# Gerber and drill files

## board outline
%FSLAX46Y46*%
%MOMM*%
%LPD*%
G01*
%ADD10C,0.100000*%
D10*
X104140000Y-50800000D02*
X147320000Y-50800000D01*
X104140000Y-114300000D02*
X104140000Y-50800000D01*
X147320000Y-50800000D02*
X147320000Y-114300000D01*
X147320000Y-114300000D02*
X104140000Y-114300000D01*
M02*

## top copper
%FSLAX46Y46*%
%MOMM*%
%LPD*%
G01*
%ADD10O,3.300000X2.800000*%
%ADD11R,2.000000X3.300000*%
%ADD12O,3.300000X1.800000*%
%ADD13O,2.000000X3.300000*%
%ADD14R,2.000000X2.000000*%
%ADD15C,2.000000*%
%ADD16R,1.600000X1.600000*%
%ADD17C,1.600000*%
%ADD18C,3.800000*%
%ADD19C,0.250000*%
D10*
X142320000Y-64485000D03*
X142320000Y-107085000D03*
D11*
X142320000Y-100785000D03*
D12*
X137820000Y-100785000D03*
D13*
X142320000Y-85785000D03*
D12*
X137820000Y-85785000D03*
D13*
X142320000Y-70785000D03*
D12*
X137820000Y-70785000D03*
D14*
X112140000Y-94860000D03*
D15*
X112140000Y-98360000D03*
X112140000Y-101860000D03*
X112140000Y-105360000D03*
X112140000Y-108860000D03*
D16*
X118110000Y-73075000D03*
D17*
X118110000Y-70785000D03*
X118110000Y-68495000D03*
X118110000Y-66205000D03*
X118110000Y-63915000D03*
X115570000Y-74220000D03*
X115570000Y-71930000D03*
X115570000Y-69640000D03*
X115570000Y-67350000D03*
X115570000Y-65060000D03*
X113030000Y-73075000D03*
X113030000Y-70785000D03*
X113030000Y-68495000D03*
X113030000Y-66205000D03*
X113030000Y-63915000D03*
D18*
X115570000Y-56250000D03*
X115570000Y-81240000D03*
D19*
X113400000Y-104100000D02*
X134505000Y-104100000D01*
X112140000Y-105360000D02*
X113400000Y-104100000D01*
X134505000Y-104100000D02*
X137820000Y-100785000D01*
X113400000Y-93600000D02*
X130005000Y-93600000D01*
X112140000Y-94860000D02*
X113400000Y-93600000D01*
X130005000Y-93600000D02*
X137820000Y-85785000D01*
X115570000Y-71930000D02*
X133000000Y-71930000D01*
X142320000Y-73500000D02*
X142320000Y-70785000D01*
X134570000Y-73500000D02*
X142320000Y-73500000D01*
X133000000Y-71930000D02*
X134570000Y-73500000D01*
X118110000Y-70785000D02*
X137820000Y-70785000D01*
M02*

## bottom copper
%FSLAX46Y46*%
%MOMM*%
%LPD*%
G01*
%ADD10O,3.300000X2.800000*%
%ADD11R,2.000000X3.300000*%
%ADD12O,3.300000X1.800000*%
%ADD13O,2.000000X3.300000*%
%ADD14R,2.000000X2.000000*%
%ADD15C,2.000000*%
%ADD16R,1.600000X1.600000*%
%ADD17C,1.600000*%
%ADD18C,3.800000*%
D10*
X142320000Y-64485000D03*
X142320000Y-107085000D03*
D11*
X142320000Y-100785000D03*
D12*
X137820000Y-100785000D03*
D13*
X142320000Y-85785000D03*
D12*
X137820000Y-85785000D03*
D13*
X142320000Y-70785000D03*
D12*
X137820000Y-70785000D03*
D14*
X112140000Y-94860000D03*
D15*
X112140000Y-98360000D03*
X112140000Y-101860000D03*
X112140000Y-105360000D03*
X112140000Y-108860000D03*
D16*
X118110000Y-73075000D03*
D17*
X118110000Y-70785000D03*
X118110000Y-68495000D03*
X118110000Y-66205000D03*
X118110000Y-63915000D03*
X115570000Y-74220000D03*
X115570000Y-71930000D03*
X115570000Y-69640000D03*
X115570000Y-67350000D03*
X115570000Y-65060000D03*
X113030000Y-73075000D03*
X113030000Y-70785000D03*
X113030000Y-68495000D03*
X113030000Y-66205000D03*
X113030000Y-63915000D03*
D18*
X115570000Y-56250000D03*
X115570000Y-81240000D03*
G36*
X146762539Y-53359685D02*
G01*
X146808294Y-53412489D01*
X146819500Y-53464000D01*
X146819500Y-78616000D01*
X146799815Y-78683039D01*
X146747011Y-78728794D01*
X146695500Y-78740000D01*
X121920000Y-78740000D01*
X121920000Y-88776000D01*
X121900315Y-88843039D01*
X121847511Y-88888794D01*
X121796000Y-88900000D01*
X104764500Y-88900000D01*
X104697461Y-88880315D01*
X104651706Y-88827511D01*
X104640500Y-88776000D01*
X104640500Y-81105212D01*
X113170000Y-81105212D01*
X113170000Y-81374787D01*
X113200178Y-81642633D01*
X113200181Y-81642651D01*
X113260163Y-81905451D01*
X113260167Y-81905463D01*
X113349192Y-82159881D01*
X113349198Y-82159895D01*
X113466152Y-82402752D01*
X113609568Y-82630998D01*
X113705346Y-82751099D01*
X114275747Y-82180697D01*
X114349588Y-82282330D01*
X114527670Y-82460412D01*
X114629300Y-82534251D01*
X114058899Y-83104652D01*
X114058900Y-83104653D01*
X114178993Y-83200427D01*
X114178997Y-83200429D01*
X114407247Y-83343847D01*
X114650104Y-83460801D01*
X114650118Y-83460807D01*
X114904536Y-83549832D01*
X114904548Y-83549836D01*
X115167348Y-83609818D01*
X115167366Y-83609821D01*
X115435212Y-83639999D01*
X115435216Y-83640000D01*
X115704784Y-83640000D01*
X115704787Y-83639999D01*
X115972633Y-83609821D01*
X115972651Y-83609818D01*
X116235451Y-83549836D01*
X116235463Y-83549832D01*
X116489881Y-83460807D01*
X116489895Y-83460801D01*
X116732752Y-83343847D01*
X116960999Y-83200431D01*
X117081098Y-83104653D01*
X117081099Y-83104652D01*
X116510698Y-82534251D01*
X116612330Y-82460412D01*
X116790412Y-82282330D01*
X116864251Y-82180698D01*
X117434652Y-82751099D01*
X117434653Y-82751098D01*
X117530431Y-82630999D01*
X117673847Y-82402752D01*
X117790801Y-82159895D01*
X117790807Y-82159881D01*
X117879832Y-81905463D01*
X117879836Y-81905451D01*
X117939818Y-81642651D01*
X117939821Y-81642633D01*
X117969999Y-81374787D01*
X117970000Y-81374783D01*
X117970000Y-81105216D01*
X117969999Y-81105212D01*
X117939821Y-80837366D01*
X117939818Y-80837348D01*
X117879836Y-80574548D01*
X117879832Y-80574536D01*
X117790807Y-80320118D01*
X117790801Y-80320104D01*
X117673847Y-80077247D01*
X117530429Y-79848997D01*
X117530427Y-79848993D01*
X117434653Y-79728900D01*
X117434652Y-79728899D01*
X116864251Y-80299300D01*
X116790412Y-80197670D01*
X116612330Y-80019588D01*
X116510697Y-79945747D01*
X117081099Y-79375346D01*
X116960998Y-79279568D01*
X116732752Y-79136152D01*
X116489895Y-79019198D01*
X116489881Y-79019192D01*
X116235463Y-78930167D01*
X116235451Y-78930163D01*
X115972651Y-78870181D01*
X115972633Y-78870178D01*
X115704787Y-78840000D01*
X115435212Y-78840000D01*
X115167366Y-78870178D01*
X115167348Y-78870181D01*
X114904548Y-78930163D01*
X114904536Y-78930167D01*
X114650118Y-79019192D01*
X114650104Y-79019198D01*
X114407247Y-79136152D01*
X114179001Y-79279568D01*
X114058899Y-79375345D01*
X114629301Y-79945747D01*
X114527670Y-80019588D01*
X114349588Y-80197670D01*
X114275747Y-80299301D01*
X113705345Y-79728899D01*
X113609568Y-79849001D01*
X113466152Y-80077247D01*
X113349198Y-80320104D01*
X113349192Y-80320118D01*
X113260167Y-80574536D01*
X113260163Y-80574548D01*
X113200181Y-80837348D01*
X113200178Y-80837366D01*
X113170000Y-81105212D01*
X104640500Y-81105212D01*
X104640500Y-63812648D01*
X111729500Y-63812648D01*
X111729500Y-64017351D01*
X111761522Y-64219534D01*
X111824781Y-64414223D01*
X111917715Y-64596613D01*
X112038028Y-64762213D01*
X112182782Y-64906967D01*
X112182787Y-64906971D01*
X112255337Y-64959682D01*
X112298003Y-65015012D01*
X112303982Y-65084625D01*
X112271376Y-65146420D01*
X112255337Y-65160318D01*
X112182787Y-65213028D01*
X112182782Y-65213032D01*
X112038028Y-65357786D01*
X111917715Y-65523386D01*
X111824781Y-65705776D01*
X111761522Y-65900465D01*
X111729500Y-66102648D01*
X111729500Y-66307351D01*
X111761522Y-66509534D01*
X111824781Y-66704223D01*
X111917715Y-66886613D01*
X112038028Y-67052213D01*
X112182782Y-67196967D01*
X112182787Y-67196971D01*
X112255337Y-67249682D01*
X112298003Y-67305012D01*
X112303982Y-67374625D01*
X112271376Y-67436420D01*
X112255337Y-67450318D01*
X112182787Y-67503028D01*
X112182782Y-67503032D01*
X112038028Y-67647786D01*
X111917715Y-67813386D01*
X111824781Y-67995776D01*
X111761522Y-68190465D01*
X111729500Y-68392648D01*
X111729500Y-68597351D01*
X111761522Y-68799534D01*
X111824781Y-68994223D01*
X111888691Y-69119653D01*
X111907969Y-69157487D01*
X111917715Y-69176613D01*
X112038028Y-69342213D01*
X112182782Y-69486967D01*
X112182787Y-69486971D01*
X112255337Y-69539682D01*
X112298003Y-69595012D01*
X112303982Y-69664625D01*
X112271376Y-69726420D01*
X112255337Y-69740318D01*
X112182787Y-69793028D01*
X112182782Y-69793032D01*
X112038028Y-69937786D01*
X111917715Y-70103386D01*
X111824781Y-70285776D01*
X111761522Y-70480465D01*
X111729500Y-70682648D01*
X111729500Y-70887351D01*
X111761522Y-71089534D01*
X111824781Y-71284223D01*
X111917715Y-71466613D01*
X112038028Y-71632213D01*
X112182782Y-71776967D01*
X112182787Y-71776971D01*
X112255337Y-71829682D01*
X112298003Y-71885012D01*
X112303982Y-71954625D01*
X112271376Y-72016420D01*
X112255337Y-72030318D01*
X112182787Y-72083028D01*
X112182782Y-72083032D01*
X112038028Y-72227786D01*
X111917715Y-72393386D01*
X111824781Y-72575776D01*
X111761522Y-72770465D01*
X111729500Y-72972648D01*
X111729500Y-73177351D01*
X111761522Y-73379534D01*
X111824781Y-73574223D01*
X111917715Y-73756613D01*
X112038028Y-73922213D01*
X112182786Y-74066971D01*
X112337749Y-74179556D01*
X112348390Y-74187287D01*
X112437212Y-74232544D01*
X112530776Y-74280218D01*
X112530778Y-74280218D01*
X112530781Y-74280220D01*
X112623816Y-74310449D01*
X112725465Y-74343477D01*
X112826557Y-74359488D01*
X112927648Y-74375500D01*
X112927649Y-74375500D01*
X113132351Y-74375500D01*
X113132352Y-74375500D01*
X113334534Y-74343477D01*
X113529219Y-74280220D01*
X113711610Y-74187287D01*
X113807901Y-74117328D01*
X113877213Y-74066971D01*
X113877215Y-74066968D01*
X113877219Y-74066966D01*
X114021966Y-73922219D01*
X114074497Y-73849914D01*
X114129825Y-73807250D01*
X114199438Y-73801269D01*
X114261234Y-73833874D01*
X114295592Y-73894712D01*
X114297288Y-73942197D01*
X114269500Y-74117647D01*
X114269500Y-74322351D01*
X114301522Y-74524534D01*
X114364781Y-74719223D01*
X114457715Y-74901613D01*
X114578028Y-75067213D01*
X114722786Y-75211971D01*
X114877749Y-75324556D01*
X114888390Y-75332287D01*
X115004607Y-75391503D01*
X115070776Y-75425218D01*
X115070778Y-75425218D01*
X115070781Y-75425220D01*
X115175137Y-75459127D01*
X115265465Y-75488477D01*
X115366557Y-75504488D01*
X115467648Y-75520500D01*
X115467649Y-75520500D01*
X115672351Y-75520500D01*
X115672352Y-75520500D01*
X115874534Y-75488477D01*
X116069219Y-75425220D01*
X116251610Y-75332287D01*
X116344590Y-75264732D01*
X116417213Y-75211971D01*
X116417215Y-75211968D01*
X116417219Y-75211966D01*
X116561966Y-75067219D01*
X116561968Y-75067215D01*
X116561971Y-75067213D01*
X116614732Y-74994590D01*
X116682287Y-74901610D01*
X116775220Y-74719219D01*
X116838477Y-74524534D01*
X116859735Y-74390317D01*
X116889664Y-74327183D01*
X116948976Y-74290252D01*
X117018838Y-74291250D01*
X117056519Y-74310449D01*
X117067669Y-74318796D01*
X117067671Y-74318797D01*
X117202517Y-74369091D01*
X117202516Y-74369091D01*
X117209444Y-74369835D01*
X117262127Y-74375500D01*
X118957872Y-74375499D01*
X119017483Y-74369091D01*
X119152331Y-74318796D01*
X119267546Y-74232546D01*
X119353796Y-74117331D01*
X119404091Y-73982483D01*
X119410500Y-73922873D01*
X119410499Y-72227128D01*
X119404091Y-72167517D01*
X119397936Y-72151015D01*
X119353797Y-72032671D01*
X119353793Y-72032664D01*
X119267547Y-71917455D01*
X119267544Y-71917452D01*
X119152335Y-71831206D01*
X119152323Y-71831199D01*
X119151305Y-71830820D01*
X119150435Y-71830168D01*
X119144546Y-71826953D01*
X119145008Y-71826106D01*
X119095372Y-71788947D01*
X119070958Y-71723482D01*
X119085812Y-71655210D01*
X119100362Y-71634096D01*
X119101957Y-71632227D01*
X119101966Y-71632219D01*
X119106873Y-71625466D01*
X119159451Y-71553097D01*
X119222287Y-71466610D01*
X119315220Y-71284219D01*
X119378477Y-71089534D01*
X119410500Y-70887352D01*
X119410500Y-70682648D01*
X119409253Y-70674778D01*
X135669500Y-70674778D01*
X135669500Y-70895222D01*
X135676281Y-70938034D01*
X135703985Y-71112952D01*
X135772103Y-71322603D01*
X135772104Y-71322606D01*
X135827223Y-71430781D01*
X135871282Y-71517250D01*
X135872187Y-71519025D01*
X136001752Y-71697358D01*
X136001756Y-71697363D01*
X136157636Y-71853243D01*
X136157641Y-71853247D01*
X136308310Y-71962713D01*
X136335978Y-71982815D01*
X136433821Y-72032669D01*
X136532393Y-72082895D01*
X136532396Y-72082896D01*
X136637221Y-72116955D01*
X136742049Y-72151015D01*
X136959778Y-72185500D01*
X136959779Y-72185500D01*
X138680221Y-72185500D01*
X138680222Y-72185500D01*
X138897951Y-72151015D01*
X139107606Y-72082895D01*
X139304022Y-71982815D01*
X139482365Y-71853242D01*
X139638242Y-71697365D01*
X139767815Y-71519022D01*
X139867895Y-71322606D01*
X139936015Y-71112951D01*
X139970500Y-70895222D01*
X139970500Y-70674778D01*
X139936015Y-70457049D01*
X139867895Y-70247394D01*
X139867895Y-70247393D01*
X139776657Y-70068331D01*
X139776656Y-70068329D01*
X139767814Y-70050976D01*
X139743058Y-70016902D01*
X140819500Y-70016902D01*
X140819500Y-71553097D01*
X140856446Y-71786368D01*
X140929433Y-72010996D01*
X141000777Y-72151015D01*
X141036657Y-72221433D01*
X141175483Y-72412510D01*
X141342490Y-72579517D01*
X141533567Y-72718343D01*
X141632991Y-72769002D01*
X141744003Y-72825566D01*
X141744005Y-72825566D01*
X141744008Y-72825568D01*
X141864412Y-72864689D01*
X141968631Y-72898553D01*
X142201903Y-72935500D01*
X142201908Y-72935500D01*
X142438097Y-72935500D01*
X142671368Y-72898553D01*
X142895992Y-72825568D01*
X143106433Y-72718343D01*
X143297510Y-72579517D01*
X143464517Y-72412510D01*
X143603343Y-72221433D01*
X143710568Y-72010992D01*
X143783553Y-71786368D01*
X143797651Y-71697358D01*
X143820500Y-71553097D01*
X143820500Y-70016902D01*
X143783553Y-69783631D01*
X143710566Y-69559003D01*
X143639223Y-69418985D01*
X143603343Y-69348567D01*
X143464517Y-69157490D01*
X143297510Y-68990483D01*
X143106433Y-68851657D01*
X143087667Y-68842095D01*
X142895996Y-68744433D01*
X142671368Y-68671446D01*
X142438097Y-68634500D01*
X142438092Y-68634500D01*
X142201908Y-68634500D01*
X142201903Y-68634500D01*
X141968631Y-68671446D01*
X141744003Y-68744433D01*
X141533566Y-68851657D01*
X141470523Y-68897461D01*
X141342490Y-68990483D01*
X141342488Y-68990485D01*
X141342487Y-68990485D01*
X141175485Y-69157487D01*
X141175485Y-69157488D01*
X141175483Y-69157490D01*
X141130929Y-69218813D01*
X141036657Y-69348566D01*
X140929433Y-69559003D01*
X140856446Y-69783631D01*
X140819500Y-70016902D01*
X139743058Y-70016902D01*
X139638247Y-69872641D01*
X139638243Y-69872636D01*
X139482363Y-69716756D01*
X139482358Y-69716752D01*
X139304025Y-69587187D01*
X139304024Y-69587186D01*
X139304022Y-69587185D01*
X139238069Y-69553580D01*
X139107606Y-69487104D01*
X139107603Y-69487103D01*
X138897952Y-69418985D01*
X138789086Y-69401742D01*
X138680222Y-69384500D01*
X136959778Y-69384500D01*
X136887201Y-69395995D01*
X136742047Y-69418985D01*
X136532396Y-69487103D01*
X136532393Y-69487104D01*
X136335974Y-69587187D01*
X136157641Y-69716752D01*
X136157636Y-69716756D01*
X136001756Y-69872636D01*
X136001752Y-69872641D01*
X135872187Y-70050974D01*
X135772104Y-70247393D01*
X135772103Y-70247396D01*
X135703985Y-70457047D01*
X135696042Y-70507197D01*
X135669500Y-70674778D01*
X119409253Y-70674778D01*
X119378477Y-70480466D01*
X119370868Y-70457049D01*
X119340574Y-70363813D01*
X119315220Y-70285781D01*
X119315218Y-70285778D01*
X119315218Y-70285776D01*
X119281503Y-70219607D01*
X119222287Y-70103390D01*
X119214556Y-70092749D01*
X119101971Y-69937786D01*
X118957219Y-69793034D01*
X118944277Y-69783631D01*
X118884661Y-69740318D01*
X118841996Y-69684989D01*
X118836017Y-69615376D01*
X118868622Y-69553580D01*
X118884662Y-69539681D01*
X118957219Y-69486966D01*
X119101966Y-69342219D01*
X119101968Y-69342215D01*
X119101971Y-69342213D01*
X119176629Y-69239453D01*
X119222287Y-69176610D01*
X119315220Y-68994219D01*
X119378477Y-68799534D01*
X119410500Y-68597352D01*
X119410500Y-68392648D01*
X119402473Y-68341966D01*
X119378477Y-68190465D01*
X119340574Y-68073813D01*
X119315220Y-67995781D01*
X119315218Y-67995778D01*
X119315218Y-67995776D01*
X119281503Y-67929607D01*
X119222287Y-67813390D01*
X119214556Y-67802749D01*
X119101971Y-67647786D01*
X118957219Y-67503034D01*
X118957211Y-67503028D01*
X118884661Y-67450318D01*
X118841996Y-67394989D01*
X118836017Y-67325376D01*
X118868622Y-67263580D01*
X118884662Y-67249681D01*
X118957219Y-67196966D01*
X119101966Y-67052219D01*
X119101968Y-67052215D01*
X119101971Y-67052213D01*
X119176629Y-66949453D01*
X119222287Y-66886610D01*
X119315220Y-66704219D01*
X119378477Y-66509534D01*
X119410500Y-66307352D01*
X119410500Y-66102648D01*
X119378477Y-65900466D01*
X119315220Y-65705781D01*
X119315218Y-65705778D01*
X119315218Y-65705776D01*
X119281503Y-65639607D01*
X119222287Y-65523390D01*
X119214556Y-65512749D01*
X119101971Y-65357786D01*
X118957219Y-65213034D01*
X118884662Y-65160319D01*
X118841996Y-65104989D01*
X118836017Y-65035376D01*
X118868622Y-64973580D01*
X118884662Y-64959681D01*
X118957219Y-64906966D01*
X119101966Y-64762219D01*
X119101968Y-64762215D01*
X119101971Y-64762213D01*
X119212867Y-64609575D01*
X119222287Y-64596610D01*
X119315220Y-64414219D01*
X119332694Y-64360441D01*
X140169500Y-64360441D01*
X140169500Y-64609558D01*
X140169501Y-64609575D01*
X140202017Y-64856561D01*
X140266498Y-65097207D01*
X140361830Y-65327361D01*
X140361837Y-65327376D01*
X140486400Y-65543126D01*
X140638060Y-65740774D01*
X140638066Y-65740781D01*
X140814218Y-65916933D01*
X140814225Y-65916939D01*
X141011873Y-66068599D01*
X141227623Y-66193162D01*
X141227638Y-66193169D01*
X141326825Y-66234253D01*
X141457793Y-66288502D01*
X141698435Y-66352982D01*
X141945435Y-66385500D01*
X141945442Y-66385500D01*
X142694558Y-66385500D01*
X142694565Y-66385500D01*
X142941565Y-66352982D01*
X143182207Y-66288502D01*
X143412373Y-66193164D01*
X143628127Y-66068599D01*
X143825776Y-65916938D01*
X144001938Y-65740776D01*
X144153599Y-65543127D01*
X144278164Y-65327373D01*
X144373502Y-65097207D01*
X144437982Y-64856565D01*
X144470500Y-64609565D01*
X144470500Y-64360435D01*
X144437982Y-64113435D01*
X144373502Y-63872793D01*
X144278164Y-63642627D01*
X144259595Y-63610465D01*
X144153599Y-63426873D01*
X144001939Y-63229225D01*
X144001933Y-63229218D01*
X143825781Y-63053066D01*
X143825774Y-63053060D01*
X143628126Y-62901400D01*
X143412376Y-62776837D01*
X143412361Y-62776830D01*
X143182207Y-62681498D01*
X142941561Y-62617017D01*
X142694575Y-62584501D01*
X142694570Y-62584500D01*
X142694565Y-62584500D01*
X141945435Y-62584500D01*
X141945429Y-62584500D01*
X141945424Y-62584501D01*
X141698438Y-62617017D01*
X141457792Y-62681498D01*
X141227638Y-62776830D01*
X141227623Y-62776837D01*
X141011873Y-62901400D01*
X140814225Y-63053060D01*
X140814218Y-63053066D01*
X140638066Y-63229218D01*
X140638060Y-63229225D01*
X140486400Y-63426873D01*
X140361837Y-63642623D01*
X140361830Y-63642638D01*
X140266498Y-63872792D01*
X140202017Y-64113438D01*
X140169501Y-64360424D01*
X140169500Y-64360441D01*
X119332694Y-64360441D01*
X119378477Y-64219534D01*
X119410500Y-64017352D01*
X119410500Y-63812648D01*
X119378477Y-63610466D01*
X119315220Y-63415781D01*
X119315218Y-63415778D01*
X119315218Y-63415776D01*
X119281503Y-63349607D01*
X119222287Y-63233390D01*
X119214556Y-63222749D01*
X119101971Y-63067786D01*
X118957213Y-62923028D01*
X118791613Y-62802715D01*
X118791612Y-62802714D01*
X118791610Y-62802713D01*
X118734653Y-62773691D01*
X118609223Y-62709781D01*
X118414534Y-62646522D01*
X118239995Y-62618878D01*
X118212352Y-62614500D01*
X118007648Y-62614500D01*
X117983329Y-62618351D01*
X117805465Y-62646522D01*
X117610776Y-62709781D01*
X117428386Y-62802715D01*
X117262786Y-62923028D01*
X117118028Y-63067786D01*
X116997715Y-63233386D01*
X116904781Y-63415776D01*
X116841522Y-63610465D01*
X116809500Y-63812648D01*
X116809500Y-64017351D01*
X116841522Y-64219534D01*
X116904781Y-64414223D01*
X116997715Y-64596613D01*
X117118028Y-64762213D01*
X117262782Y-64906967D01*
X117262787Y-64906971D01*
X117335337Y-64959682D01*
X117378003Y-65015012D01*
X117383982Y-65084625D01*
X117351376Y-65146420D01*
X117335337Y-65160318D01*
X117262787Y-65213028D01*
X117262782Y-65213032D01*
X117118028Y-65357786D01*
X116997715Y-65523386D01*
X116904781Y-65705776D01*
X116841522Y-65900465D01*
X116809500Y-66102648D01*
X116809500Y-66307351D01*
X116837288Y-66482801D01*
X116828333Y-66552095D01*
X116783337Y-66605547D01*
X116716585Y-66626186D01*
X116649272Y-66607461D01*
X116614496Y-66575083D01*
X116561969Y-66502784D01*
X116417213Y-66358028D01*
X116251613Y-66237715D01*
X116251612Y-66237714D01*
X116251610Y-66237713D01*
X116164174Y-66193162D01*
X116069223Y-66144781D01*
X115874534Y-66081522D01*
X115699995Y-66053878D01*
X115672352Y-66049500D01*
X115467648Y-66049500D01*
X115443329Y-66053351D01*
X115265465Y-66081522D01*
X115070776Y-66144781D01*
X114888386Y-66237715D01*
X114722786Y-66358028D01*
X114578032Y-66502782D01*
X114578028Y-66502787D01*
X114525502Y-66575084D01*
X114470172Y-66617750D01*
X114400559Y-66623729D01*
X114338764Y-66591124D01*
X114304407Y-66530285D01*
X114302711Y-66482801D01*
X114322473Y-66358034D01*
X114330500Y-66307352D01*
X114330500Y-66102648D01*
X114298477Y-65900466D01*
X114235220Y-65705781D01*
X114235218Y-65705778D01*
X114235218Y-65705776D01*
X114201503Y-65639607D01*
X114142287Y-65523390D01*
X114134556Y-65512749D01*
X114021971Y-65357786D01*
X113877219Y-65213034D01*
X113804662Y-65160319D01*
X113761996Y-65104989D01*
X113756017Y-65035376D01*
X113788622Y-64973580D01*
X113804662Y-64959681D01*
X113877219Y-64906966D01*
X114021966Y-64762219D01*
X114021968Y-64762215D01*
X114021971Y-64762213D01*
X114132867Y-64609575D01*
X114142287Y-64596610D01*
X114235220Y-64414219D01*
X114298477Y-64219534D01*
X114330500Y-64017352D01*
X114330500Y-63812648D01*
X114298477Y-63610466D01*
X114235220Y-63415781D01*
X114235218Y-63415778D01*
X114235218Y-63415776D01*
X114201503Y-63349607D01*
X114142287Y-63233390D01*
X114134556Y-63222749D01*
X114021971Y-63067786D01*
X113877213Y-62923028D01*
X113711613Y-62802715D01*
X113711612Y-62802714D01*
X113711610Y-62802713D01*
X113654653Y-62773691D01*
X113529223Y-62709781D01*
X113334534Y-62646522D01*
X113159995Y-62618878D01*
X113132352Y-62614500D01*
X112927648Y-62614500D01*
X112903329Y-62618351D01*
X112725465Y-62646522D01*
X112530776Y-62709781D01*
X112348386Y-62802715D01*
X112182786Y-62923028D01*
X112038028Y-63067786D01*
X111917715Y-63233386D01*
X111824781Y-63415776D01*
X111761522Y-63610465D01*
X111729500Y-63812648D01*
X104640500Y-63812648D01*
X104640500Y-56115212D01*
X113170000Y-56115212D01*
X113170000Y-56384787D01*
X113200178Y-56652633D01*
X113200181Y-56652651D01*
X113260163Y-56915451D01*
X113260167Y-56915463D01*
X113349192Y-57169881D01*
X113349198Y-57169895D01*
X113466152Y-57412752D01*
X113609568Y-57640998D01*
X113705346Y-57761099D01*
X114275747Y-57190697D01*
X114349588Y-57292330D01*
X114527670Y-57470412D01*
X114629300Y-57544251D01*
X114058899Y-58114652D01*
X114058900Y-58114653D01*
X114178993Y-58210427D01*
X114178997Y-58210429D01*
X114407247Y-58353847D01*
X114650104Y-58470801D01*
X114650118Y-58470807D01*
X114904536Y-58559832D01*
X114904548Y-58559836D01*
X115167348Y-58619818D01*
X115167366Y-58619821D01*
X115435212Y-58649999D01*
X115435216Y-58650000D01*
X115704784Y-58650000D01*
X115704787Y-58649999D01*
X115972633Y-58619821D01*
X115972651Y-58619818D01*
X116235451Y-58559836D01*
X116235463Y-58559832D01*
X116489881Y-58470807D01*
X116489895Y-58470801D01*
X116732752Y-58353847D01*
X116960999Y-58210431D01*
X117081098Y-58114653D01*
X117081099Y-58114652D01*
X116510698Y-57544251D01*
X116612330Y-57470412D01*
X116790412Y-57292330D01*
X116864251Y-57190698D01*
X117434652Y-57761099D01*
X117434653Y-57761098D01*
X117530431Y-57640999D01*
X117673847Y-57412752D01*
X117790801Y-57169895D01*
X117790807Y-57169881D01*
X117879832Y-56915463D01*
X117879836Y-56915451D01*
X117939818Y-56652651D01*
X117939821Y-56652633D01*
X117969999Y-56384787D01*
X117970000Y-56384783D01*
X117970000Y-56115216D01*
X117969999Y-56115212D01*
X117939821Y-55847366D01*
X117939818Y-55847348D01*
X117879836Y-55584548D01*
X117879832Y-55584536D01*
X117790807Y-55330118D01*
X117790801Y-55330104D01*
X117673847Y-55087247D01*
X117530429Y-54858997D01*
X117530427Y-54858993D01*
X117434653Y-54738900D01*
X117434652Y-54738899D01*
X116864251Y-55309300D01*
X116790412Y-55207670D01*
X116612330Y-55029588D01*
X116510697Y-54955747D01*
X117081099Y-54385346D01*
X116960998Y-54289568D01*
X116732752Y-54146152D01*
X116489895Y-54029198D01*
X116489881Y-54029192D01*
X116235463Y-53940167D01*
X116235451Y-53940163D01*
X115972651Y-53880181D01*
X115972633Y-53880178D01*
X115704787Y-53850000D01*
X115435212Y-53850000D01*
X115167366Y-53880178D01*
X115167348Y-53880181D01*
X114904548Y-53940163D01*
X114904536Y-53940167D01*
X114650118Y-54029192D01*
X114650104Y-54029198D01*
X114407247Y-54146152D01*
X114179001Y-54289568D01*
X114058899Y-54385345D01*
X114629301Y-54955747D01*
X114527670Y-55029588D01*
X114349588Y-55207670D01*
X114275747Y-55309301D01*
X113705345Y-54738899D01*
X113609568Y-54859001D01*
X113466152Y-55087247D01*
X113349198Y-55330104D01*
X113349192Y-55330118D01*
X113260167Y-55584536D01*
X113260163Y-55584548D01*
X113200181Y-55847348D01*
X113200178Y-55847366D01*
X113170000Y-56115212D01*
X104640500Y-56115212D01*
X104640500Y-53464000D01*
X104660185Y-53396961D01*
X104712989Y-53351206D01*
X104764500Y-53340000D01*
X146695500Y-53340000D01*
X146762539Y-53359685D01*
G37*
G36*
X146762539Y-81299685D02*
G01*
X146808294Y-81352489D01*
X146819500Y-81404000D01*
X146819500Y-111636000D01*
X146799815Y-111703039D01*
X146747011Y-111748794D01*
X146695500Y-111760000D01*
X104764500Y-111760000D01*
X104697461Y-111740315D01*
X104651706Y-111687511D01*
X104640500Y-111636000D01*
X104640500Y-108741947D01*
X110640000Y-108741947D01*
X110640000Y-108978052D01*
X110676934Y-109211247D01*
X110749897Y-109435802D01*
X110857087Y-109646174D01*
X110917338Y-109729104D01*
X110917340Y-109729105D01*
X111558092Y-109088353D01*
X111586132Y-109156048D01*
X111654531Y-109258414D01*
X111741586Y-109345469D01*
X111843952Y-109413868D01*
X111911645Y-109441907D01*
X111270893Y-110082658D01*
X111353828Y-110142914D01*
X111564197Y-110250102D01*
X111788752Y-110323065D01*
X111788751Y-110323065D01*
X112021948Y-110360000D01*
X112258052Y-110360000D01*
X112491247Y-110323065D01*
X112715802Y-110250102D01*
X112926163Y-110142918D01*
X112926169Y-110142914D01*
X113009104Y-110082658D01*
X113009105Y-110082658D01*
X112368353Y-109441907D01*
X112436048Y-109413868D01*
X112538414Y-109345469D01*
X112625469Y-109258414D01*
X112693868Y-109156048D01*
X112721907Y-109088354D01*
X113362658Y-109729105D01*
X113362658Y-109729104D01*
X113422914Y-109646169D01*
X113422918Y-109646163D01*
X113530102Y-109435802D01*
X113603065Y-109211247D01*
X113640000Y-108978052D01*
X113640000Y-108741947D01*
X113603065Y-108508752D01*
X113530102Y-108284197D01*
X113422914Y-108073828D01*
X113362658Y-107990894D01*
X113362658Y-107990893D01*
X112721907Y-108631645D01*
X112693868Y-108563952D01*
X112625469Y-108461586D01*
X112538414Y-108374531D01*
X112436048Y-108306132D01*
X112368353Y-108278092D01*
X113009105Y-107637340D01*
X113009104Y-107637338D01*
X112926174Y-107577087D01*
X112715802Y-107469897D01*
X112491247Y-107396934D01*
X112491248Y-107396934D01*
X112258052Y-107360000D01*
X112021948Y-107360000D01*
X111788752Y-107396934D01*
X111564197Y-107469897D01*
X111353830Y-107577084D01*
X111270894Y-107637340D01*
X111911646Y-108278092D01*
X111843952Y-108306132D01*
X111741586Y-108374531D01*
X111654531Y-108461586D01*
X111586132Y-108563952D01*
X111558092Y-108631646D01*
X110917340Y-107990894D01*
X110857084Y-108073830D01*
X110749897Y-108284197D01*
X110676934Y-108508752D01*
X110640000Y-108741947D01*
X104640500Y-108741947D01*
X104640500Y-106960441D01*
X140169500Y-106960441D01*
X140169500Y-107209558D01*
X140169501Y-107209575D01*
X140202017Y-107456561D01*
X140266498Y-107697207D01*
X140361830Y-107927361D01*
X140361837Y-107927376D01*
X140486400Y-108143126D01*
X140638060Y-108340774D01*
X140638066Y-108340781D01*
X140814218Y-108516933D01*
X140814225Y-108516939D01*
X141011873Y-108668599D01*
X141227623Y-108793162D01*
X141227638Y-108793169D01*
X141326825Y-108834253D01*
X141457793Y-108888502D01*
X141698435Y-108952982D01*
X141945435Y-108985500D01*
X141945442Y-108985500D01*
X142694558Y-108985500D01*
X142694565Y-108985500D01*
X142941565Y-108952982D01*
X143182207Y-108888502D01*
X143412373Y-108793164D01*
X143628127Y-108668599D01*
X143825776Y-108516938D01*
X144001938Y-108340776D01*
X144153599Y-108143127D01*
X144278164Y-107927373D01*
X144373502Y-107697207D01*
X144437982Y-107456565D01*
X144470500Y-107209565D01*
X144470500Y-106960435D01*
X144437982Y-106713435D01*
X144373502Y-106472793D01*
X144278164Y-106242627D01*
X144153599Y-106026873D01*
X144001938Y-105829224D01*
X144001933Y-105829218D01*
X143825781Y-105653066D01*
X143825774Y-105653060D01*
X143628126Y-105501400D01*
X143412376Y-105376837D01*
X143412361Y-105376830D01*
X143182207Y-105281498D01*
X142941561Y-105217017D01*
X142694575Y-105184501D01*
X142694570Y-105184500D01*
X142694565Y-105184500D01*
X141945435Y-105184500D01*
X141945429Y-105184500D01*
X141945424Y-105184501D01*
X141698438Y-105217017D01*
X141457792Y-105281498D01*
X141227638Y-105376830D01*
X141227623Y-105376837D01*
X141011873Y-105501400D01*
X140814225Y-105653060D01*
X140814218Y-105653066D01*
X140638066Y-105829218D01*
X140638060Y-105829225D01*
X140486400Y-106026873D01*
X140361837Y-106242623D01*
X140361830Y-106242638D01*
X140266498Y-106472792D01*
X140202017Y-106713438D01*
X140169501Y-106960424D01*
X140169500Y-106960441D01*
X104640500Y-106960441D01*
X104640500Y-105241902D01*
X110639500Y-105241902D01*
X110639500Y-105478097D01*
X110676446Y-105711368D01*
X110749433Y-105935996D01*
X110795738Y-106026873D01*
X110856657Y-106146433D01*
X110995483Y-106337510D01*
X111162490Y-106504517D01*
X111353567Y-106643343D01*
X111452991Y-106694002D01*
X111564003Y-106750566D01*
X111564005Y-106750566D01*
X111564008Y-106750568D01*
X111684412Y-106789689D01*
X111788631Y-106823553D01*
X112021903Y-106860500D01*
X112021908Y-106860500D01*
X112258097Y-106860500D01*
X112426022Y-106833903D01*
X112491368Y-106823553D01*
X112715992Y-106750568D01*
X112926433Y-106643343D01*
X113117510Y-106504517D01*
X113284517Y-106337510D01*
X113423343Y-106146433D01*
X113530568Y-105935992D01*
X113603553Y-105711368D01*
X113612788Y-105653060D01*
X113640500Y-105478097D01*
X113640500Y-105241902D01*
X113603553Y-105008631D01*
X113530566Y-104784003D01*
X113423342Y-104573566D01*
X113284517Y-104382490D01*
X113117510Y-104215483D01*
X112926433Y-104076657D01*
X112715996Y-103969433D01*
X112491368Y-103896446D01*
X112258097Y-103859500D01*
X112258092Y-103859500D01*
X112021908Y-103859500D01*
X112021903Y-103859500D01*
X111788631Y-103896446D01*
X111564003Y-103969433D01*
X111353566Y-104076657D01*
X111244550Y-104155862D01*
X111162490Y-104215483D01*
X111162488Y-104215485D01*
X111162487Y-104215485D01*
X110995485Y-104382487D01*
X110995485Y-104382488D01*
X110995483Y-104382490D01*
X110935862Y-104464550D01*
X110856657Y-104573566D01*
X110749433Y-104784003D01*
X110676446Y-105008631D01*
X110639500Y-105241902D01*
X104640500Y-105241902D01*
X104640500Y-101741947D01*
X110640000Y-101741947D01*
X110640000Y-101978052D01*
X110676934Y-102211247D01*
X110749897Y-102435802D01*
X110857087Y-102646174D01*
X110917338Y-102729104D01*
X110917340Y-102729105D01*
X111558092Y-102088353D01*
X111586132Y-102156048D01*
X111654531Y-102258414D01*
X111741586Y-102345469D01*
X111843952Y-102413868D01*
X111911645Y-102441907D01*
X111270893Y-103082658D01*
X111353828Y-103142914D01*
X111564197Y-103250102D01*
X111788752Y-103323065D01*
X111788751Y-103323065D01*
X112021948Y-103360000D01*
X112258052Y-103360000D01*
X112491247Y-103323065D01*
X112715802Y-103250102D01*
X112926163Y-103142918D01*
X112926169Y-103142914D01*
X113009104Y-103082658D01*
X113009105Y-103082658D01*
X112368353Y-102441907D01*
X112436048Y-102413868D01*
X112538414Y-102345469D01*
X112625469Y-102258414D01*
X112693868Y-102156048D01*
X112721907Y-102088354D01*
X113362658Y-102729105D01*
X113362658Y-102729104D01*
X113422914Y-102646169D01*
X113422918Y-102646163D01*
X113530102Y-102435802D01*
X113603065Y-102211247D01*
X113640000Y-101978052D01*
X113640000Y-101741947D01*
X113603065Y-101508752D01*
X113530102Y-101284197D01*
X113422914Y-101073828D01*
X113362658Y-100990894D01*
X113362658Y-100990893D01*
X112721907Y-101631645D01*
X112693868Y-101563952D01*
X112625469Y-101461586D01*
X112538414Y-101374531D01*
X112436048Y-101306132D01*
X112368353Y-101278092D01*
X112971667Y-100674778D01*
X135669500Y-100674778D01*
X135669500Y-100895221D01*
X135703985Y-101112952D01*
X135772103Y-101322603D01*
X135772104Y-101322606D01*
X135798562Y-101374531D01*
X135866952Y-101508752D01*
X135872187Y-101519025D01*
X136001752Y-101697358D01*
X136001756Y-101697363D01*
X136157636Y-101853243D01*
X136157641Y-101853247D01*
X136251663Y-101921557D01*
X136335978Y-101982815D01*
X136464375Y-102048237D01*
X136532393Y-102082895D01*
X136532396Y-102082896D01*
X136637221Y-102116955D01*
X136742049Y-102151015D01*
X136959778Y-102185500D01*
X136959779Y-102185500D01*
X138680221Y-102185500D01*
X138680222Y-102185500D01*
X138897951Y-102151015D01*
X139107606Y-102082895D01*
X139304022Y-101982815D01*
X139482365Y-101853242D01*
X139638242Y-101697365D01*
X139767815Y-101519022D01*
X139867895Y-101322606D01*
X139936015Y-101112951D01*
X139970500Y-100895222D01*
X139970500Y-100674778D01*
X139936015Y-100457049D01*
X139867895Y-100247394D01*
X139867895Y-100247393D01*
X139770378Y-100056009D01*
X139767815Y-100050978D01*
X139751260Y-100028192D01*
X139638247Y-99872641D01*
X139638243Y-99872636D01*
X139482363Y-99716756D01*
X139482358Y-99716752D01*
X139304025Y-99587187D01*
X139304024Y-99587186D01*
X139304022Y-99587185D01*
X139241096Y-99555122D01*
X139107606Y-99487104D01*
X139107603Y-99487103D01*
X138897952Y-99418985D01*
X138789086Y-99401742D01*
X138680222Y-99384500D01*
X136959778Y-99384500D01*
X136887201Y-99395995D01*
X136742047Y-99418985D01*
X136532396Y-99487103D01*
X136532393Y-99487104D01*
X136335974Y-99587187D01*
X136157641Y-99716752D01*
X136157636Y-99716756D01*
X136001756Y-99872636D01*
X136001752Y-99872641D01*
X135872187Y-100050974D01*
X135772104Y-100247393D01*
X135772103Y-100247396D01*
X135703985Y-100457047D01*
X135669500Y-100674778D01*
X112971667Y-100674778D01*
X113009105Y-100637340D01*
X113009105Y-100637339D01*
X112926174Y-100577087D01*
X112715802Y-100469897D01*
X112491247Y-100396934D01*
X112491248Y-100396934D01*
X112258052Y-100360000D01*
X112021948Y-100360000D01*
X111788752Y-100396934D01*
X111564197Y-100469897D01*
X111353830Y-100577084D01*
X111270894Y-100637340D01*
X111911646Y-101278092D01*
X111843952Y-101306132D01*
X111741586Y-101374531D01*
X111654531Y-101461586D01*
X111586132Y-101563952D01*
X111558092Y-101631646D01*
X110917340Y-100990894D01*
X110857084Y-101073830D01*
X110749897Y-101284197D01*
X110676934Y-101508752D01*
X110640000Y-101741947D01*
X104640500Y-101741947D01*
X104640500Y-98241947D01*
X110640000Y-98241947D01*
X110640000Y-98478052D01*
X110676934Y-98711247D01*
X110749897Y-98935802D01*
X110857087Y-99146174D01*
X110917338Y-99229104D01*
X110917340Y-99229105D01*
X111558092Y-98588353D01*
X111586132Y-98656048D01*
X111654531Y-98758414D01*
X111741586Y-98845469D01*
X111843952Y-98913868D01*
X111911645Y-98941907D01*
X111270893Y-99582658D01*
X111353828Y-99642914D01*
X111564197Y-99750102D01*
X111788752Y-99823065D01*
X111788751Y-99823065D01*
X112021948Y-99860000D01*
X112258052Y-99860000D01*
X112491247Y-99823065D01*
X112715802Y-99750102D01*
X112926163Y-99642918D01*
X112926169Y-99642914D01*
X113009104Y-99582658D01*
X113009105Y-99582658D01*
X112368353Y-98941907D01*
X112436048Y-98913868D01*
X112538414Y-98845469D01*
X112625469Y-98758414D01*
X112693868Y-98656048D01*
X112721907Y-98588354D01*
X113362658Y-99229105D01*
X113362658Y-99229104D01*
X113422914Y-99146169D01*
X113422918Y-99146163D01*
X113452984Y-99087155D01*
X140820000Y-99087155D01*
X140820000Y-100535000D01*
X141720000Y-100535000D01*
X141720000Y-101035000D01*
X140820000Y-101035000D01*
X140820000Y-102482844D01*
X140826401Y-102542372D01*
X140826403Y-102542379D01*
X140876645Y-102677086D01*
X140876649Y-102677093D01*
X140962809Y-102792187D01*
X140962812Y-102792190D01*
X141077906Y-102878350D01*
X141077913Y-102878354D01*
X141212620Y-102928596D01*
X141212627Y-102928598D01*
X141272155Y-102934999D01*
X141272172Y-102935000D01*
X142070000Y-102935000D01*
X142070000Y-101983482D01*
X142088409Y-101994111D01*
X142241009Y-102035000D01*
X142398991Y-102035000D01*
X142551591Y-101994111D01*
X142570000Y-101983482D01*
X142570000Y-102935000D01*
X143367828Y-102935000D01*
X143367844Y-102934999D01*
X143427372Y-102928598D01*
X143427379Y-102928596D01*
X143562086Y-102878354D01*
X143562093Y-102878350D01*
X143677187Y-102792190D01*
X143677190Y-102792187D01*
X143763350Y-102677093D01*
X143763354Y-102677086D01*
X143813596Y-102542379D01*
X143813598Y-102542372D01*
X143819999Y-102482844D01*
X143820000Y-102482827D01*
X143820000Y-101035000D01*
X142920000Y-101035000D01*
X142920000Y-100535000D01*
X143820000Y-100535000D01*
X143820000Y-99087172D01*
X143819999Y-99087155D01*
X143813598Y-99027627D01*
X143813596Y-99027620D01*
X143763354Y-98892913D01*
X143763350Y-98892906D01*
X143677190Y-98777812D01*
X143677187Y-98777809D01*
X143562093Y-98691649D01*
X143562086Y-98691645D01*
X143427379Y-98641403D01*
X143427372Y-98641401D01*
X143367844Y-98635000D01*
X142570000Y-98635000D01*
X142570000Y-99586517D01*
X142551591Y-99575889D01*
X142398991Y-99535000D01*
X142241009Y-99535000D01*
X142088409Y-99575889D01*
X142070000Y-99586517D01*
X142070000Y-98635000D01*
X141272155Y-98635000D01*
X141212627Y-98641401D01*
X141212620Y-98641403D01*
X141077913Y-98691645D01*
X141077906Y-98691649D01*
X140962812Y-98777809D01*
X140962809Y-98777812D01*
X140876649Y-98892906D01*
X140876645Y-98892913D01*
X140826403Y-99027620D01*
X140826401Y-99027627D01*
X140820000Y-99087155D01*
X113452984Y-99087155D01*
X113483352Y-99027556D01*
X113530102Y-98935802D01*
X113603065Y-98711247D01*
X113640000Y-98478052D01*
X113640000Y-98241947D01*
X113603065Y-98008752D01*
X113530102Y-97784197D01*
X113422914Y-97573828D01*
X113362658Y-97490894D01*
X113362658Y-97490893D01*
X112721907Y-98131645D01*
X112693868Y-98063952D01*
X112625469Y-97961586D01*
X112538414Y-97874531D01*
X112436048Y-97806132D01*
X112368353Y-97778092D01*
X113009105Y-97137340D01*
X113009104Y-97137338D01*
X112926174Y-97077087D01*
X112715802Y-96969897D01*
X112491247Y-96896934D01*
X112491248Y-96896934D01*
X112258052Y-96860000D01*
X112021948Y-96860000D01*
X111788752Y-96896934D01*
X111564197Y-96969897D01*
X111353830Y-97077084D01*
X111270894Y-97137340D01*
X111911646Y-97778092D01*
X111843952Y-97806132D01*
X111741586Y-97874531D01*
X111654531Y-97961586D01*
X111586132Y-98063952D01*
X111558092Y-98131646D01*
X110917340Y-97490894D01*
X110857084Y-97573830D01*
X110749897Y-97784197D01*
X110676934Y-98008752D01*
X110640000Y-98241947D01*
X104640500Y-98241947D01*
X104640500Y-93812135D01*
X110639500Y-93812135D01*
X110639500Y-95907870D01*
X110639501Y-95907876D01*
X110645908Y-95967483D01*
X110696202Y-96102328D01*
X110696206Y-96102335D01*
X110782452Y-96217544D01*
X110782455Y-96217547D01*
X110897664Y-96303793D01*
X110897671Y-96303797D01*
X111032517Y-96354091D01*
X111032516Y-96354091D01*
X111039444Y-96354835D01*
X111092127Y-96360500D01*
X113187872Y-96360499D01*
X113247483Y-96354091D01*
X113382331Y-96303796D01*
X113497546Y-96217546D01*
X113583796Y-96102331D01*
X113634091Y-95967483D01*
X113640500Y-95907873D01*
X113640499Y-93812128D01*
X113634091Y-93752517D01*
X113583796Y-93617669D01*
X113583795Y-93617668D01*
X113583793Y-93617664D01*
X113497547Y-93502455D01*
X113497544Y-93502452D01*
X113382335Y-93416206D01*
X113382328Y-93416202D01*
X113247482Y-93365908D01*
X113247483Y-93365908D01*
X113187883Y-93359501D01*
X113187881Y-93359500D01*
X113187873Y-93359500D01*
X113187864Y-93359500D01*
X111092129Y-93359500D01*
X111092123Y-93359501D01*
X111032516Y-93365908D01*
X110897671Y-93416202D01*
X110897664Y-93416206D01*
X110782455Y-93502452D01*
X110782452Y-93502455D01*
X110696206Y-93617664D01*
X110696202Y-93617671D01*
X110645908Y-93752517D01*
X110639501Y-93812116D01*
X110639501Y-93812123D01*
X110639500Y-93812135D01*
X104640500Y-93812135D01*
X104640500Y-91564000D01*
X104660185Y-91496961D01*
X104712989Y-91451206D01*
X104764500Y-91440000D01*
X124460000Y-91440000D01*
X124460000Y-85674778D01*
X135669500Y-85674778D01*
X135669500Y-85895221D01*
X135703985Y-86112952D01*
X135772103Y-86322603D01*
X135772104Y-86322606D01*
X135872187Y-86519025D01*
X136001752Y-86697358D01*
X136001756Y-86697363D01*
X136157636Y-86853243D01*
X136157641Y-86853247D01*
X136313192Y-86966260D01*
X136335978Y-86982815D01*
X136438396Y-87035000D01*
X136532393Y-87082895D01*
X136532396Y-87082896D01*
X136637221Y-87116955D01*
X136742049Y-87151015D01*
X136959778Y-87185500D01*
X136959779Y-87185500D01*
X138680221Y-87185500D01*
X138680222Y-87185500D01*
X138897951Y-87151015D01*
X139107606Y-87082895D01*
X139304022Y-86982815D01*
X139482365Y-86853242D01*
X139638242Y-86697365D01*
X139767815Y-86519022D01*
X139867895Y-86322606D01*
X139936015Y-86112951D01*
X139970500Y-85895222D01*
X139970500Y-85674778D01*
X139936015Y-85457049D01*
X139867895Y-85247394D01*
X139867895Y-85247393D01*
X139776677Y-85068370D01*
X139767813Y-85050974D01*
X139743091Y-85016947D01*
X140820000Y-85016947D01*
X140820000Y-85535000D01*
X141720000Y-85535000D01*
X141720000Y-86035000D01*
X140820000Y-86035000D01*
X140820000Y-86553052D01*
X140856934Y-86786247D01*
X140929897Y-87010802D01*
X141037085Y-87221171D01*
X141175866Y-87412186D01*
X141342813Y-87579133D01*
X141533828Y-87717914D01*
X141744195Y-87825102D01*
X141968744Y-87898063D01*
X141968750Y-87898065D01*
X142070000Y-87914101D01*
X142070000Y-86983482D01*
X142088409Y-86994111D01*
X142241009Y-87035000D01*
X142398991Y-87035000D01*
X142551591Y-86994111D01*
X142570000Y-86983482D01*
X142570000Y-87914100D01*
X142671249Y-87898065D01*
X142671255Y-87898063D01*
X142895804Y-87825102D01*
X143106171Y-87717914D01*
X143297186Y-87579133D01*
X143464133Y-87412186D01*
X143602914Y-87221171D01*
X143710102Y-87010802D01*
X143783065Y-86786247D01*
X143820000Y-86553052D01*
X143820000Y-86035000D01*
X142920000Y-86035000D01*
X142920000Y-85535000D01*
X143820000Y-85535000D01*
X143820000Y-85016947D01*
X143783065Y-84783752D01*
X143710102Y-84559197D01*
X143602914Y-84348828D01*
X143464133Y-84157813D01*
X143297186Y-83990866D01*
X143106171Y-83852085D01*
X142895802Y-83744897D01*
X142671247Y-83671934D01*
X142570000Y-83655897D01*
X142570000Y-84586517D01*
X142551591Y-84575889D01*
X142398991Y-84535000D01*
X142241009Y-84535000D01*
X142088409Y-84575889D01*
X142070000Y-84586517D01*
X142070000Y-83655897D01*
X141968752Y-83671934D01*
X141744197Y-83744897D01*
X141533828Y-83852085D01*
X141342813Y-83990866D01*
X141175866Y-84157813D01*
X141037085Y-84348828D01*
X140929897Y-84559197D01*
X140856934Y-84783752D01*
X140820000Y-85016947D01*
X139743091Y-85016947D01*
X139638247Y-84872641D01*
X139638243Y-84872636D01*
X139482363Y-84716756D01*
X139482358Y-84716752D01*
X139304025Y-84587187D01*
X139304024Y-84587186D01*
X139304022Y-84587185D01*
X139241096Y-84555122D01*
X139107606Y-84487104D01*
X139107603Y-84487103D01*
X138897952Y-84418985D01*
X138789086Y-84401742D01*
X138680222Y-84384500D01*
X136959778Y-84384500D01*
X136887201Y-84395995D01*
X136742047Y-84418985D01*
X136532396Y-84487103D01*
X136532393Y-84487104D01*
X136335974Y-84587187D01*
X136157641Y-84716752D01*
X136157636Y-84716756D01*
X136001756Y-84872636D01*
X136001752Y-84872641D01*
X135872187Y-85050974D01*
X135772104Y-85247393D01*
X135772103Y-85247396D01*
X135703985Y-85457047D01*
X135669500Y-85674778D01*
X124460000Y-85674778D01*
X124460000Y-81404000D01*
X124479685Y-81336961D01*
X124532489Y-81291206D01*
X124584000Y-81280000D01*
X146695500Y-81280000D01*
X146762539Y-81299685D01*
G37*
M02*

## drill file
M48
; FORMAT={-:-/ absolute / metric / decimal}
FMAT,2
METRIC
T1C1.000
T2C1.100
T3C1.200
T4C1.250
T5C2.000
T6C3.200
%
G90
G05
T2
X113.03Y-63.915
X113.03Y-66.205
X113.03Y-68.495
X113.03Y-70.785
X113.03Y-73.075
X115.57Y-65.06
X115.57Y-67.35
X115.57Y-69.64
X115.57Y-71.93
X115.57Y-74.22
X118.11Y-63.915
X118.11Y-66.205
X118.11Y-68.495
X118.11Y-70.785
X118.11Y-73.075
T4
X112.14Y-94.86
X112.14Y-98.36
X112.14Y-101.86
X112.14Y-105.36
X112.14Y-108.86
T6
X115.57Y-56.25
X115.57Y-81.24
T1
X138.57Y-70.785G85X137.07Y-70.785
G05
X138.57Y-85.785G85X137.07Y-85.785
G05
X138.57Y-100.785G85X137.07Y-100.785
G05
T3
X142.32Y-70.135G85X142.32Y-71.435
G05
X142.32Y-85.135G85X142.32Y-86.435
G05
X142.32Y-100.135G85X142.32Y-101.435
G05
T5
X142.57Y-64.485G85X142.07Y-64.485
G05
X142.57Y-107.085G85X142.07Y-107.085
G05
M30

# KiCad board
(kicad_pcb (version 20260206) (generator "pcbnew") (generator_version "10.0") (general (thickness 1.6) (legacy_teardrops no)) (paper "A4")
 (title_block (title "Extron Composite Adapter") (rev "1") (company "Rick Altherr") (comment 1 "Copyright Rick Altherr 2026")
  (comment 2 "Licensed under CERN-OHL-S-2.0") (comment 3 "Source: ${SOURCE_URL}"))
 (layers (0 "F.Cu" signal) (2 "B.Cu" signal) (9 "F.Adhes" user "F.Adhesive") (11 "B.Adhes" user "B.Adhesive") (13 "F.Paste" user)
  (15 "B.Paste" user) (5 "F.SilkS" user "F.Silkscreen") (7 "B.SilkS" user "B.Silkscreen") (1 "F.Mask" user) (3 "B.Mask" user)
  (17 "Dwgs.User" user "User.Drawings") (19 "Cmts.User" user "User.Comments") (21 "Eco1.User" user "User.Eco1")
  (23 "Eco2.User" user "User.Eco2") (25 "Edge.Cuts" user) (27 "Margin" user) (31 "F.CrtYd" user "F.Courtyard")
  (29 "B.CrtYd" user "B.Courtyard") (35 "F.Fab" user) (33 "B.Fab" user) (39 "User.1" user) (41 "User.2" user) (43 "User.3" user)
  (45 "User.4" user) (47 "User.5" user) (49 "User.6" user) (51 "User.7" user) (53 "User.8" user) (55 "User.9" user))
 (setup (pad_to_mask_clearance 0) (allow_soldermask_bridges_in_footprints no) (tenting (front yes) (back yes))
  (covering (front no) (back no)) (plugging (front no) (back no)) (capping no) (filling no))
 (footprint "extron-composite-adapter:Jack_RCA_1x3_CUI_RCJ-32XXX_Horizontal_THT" (layer "F.Cu") (at 142.32 100.785 -90)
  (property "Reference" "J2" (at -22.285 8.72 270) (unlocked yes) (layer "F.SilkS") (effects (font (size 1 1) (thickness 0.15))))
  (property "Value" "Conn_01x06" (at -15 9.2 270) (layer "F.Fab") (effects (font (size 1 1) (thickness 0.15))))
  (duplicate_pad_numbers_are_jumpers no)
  (pad "" thru_hole oval (at -36.3 0 270) (size 2.8 3.3) (drill oval 2 2.5) (layers "*.Cu" "*.Mask") (remove_unused_layers no))
  (pad "" thru_hole oval (at 6.3 0 270) (size 2.8 3.3) (drill oval 2 2.5) (layers "*.Cu" "*.Mask") (remove_unused_layers no))
  (pad "1" thru_hole rect (at 0 0 270) (size 3.3 2) (drill oval 2.5 1.2) (layers "*.Cu" "*.Mask") (remove_unused_layers no)
   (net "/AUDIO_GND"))
  (pad "2" thru_hole oval (at 0 4.5 270) (size 1.8 3.3) (drill oval 1 2.5) (layers "*.Cu" "*.Mask") (remove_unused_layers no)
   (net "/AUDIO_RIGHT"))
  (pad "3" thru_hole oval (at -15 0 270) (size 3.3 2) (drill oval 2.5 1.2) (layers "*.Cu" "*.Mask") (remove_unused_layers no)
   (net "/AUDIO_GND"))
  (pad "4" thru_hole oval (at -15 4.5 270) (size 1.8 3.3) (drill oval 1 2.5) (layers "*.Cu" "*.Mask") (remove_unused_layers no)
   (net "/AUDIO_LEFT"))
  (pad "5" thru_hole oval (at -30 0 270) (size 3.3 2) (drill oval 2.5 1.2) (layers "*.Cu" "*.Mask") (remove_unused_layers no)
   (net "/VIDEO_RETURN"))
  (pad "6" thru_hole oval (at -30 4.5 270) (size 1.8 3.3) (drill oval 1 2.5) (layers "*.Cu" "*.Mask") (remove_unused_layers no)
   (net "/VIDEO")))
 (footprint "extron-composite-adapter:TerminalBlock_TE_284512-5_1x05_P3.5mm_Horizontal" (layer "F.Cu") (at 112.14 94.86 -90)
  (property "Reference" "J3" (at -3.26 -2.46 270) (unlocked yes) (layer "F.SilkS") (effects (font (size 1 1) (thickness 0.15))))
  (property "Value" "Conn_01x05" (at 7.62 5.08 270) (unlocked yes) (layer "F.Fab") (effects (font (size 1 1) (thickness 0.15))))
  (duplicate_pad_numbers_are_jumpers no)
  (pad "1" thru_hole rect (at 0 0 270) (size 2 2) (drill 1.25) (layers "*.Cu" "*.Mask") (remove_unused_layers no) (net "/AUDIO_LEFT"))
  (pad "2" thru_hole circle (at 3.5 0 270) (size 2 2) (drill 1.25) (layers "*.Cu" "*.Mask") (remove_unused_layers no) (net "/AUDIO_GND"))
  (pad "3" thru_hole circle (at 7 0 270) (size 2 2) (drill 1.25) (layers "*.Cu" "*.Mask") (remove_unused_layers no) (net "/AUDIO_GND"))
  (pad "4" thru_hole circle (at 10.5 0 270) (size 2 2) (drill 1.25) (layers "*.Cu" "*.Mask") (remove_unused_layers no) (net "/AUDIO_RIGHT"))
  (pad "5" thru_hole circle (at 14 0 270) (size 2 2) (drill 1.25) (layers "*.Cu" "*.Mask") (remove_unused_layers no) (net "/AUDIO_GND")))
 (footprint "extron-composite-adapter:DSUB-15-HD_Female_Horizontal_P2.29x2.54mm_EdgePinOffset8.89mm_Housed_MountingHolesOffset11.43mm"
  (layer "F.Cu") (at 118.11 73.075 -90)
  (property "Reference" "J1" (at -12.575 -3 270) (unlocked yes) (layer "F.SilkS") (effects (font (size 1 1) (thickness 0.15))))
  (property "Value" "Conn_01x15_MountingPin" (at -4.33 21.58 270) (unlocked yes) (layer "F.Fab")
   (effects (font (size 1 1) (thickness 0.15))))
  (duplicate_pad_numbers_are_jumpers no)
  (pad "1" thru_hole rect (at 0 0 270) (size 1.6 1.6) (drill 1.1) (layers "*.Cu" "*.Mask") (remove_unused_layers no)
   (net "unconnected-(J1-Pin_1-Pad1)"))
  (pad "2" thru_hole circle (at -2.29 0 270) (size 1.6 1.6) (drill 1.1) (layers "*.Cu" "*.Mask") (remove_unused_layers no) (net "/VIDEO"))
  (pad "3" thru_hole circle (at -4.58 0 270) (size 1.6 1.6) (drill 1.1) (layers "*.Cu" "*.Mask") (remove_unused_layers no)
   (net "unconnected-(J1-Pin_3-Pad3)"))
  (pad "4" thru_hole circle (at -6.87 0 270) (size 1.6 1.6) (drill 1.1) (layers "*.Cu" "*.Mask") (remove_unused_layers no)
   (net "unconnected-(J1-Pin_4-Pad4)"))
  (pad "5" thru_hole circle (at -9.16 0 270) (size 1.6 1.6) (drill 1.1) (layers "*.Cu" "*.Mask") (remove_unused_layers no)
   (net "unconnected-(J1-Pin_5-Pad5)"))
  (pad "6" thru_hole circle (at 1.145 2.54 270) (size 1.6 1.6) (drill 1.1) (layers "*.Cu" "*.Mask") (remove_unused_layers no)
   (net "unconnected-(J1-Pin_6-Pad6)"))
  (pad "7" thru_hole circle (at -1.145 2.54 270) (size 1.6 1.6) (drill 1.1) (layers "*.Cu" "*.Mask") (remove_unused_layers no)
   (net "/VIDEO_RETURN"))
  (pad "8" thru_hole circle (at -3.435 2.54 270) (size 1.6 1.6) (drill 1.1) (layers "*.Cu" "*.Mask") (remove_unused_layers no)
   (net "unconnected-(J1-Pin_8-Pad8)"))
  (pad "9" thru_hole circle (at -5.725 2.54 270) (size 1.6 1.6) (drill 1.1) (layers "*.Cu" "*.Mask") (remove_unused_layers no)
   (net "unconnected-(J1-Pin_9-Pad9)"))
  (pad "10" thru_hole circle (at -8.015 2.54 270) (size 1.6 1.6) (drill 1.1) (layers "*.Cu" "*.Mask") (remove_unused_layers no) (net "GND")
   (zone_connect 2))
  (pad "11" thru_hole circle (at 0 5.08 270) (size 1.6 1.6) (drill 1.1) (layers "*.Cu" "*.Mask") (remove_unused_layers no)
   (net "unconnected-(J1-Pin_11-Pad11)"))
  (pad "12" thru_hole circle (at -2.29 5.08 270) (size 1.6 1.6) (drill 1.1) (layers "*.Cu" "*.Mask") (remove_unused_layers no)
   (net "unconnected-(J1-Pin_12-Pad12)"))
  (pad "13" thru_hole circle (at -4.58 5.08 270) (size 1.6 1.6) (drill 1.1) (layers "*.Cu" "*.Mask") (remove_unused_layers no)
   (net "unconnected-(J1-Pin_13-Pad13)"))
  (pad "14" thru_hole circle (at -6.87 5.08 270) (size 1.6 1.6) (drill 1.1) (layers "*.Cu" "*.Mask") (remove_unused_layers no)
   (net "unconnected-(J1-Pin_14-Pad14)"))
  (pad "15" thru_hole circle (at -9.16 5.08 270) (size 1.6 1.6) (drill 1.1) (layers "*.Cu" "*.Mask") (remove_unused_layers no)
   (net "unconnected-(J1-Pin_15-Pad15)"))
  (pad "MP" thru_hole circle (at -16.825 2.54 270) (size 3.8 3.8) (drill 3.2) (layers "*.Cu" "*.Mask") (remove_unused_layers no) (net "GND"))
  (pad "MP" thru_hole circle (at 8.165 2.54 270) (size 3.8 3.8) (drill 3.2) (layers "*.Cu" "*.Mask") (remove_unused_layers no) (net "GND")))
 (gr_line (start 104.14 50.8) (end 147.32 50.8) (stroke (width 0.1) (type default)) (layer "Edge.Cuts"))
 (gr_line (start 104.14 114.3) (end 104.14 50.8) (stroke (width 0.1) (type default)) (layer "Edge.Cuts"))
 (gr_line (start 147.32 50.8) (end 147.32 114.3) (stroke (width 0.1) (type default)) (layer "Edge.Cuts"))
 (gr_line (start 147.32 114.3) (end 104.14 114.3) (stroke (width 0.1) (type default)) (layer "Edge.Cuts"))
 (segment (start 113.4 104.1) (end 134.505 104.1) (width 0.25) (layer "F.Cu") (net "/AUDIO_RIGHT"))
 (segment (start 112.14 105.36) (end 113.4 104.1) (width 0.25) (layer "F.Cu") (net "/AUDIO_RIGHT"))
 (segment (start 134.505 104.1) (end 137.82 100.785) (width 0.25) (layer "F.Cu") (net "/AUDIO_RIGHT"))
 (segment (start 113.4 93.6) (end 130.005 93.6) (width 0.25) (layer "F.Cu") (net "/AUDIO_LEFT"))
 (segment (start 112.14 94.86) (end 113.4 93.6) (width 0.25) (layer "F.Cu") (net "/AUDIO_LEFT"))
 (segment (start 130.005 93.6) (end 137.82 85.785) (width 0.25) (layer "F.Cu") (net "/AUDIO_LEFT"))
 (segment (start 115.57 71.93) (end 133 71.93) (width 0.25) (layer "F.Cu") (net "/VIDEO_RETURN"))
 (segment (start 142.32 73.5) (end 142.32 70.785) (width 0.25) (layer "F.Cu") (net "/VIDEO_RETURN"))
 (segment (start 134.57 73.5) (end 142.32 73.5) (width 0.25) (layer "F.Cu") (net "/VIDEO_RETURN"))
 (segment (start 133 71.93) (end 134.57 73.5) (width 0.25) (layer "F.Cu") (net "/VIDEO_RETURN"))
 (segment (start 118.11 70.785) (end 137.82 70.785) (width 0.25) (layer "F.Cu") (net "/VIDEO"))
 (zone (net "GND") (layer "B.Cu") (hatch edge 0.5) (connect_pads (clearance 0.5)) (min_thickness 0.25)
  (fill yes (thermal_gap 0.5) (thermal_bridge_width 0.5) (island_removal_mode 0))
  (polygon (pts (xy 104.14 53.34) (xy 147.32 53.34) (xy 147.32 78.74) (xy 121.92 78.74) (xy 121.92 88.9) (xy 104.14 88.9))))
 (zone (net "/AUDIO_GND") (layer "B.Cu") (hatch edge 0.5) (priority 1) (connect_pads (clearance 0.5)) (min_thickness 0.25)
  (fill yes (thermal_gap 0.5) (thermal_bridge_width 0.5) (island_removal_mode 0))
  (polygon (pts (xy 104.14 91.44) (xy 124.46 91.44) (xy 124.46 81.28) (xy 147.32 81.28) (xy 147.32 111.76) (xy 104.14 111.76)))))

